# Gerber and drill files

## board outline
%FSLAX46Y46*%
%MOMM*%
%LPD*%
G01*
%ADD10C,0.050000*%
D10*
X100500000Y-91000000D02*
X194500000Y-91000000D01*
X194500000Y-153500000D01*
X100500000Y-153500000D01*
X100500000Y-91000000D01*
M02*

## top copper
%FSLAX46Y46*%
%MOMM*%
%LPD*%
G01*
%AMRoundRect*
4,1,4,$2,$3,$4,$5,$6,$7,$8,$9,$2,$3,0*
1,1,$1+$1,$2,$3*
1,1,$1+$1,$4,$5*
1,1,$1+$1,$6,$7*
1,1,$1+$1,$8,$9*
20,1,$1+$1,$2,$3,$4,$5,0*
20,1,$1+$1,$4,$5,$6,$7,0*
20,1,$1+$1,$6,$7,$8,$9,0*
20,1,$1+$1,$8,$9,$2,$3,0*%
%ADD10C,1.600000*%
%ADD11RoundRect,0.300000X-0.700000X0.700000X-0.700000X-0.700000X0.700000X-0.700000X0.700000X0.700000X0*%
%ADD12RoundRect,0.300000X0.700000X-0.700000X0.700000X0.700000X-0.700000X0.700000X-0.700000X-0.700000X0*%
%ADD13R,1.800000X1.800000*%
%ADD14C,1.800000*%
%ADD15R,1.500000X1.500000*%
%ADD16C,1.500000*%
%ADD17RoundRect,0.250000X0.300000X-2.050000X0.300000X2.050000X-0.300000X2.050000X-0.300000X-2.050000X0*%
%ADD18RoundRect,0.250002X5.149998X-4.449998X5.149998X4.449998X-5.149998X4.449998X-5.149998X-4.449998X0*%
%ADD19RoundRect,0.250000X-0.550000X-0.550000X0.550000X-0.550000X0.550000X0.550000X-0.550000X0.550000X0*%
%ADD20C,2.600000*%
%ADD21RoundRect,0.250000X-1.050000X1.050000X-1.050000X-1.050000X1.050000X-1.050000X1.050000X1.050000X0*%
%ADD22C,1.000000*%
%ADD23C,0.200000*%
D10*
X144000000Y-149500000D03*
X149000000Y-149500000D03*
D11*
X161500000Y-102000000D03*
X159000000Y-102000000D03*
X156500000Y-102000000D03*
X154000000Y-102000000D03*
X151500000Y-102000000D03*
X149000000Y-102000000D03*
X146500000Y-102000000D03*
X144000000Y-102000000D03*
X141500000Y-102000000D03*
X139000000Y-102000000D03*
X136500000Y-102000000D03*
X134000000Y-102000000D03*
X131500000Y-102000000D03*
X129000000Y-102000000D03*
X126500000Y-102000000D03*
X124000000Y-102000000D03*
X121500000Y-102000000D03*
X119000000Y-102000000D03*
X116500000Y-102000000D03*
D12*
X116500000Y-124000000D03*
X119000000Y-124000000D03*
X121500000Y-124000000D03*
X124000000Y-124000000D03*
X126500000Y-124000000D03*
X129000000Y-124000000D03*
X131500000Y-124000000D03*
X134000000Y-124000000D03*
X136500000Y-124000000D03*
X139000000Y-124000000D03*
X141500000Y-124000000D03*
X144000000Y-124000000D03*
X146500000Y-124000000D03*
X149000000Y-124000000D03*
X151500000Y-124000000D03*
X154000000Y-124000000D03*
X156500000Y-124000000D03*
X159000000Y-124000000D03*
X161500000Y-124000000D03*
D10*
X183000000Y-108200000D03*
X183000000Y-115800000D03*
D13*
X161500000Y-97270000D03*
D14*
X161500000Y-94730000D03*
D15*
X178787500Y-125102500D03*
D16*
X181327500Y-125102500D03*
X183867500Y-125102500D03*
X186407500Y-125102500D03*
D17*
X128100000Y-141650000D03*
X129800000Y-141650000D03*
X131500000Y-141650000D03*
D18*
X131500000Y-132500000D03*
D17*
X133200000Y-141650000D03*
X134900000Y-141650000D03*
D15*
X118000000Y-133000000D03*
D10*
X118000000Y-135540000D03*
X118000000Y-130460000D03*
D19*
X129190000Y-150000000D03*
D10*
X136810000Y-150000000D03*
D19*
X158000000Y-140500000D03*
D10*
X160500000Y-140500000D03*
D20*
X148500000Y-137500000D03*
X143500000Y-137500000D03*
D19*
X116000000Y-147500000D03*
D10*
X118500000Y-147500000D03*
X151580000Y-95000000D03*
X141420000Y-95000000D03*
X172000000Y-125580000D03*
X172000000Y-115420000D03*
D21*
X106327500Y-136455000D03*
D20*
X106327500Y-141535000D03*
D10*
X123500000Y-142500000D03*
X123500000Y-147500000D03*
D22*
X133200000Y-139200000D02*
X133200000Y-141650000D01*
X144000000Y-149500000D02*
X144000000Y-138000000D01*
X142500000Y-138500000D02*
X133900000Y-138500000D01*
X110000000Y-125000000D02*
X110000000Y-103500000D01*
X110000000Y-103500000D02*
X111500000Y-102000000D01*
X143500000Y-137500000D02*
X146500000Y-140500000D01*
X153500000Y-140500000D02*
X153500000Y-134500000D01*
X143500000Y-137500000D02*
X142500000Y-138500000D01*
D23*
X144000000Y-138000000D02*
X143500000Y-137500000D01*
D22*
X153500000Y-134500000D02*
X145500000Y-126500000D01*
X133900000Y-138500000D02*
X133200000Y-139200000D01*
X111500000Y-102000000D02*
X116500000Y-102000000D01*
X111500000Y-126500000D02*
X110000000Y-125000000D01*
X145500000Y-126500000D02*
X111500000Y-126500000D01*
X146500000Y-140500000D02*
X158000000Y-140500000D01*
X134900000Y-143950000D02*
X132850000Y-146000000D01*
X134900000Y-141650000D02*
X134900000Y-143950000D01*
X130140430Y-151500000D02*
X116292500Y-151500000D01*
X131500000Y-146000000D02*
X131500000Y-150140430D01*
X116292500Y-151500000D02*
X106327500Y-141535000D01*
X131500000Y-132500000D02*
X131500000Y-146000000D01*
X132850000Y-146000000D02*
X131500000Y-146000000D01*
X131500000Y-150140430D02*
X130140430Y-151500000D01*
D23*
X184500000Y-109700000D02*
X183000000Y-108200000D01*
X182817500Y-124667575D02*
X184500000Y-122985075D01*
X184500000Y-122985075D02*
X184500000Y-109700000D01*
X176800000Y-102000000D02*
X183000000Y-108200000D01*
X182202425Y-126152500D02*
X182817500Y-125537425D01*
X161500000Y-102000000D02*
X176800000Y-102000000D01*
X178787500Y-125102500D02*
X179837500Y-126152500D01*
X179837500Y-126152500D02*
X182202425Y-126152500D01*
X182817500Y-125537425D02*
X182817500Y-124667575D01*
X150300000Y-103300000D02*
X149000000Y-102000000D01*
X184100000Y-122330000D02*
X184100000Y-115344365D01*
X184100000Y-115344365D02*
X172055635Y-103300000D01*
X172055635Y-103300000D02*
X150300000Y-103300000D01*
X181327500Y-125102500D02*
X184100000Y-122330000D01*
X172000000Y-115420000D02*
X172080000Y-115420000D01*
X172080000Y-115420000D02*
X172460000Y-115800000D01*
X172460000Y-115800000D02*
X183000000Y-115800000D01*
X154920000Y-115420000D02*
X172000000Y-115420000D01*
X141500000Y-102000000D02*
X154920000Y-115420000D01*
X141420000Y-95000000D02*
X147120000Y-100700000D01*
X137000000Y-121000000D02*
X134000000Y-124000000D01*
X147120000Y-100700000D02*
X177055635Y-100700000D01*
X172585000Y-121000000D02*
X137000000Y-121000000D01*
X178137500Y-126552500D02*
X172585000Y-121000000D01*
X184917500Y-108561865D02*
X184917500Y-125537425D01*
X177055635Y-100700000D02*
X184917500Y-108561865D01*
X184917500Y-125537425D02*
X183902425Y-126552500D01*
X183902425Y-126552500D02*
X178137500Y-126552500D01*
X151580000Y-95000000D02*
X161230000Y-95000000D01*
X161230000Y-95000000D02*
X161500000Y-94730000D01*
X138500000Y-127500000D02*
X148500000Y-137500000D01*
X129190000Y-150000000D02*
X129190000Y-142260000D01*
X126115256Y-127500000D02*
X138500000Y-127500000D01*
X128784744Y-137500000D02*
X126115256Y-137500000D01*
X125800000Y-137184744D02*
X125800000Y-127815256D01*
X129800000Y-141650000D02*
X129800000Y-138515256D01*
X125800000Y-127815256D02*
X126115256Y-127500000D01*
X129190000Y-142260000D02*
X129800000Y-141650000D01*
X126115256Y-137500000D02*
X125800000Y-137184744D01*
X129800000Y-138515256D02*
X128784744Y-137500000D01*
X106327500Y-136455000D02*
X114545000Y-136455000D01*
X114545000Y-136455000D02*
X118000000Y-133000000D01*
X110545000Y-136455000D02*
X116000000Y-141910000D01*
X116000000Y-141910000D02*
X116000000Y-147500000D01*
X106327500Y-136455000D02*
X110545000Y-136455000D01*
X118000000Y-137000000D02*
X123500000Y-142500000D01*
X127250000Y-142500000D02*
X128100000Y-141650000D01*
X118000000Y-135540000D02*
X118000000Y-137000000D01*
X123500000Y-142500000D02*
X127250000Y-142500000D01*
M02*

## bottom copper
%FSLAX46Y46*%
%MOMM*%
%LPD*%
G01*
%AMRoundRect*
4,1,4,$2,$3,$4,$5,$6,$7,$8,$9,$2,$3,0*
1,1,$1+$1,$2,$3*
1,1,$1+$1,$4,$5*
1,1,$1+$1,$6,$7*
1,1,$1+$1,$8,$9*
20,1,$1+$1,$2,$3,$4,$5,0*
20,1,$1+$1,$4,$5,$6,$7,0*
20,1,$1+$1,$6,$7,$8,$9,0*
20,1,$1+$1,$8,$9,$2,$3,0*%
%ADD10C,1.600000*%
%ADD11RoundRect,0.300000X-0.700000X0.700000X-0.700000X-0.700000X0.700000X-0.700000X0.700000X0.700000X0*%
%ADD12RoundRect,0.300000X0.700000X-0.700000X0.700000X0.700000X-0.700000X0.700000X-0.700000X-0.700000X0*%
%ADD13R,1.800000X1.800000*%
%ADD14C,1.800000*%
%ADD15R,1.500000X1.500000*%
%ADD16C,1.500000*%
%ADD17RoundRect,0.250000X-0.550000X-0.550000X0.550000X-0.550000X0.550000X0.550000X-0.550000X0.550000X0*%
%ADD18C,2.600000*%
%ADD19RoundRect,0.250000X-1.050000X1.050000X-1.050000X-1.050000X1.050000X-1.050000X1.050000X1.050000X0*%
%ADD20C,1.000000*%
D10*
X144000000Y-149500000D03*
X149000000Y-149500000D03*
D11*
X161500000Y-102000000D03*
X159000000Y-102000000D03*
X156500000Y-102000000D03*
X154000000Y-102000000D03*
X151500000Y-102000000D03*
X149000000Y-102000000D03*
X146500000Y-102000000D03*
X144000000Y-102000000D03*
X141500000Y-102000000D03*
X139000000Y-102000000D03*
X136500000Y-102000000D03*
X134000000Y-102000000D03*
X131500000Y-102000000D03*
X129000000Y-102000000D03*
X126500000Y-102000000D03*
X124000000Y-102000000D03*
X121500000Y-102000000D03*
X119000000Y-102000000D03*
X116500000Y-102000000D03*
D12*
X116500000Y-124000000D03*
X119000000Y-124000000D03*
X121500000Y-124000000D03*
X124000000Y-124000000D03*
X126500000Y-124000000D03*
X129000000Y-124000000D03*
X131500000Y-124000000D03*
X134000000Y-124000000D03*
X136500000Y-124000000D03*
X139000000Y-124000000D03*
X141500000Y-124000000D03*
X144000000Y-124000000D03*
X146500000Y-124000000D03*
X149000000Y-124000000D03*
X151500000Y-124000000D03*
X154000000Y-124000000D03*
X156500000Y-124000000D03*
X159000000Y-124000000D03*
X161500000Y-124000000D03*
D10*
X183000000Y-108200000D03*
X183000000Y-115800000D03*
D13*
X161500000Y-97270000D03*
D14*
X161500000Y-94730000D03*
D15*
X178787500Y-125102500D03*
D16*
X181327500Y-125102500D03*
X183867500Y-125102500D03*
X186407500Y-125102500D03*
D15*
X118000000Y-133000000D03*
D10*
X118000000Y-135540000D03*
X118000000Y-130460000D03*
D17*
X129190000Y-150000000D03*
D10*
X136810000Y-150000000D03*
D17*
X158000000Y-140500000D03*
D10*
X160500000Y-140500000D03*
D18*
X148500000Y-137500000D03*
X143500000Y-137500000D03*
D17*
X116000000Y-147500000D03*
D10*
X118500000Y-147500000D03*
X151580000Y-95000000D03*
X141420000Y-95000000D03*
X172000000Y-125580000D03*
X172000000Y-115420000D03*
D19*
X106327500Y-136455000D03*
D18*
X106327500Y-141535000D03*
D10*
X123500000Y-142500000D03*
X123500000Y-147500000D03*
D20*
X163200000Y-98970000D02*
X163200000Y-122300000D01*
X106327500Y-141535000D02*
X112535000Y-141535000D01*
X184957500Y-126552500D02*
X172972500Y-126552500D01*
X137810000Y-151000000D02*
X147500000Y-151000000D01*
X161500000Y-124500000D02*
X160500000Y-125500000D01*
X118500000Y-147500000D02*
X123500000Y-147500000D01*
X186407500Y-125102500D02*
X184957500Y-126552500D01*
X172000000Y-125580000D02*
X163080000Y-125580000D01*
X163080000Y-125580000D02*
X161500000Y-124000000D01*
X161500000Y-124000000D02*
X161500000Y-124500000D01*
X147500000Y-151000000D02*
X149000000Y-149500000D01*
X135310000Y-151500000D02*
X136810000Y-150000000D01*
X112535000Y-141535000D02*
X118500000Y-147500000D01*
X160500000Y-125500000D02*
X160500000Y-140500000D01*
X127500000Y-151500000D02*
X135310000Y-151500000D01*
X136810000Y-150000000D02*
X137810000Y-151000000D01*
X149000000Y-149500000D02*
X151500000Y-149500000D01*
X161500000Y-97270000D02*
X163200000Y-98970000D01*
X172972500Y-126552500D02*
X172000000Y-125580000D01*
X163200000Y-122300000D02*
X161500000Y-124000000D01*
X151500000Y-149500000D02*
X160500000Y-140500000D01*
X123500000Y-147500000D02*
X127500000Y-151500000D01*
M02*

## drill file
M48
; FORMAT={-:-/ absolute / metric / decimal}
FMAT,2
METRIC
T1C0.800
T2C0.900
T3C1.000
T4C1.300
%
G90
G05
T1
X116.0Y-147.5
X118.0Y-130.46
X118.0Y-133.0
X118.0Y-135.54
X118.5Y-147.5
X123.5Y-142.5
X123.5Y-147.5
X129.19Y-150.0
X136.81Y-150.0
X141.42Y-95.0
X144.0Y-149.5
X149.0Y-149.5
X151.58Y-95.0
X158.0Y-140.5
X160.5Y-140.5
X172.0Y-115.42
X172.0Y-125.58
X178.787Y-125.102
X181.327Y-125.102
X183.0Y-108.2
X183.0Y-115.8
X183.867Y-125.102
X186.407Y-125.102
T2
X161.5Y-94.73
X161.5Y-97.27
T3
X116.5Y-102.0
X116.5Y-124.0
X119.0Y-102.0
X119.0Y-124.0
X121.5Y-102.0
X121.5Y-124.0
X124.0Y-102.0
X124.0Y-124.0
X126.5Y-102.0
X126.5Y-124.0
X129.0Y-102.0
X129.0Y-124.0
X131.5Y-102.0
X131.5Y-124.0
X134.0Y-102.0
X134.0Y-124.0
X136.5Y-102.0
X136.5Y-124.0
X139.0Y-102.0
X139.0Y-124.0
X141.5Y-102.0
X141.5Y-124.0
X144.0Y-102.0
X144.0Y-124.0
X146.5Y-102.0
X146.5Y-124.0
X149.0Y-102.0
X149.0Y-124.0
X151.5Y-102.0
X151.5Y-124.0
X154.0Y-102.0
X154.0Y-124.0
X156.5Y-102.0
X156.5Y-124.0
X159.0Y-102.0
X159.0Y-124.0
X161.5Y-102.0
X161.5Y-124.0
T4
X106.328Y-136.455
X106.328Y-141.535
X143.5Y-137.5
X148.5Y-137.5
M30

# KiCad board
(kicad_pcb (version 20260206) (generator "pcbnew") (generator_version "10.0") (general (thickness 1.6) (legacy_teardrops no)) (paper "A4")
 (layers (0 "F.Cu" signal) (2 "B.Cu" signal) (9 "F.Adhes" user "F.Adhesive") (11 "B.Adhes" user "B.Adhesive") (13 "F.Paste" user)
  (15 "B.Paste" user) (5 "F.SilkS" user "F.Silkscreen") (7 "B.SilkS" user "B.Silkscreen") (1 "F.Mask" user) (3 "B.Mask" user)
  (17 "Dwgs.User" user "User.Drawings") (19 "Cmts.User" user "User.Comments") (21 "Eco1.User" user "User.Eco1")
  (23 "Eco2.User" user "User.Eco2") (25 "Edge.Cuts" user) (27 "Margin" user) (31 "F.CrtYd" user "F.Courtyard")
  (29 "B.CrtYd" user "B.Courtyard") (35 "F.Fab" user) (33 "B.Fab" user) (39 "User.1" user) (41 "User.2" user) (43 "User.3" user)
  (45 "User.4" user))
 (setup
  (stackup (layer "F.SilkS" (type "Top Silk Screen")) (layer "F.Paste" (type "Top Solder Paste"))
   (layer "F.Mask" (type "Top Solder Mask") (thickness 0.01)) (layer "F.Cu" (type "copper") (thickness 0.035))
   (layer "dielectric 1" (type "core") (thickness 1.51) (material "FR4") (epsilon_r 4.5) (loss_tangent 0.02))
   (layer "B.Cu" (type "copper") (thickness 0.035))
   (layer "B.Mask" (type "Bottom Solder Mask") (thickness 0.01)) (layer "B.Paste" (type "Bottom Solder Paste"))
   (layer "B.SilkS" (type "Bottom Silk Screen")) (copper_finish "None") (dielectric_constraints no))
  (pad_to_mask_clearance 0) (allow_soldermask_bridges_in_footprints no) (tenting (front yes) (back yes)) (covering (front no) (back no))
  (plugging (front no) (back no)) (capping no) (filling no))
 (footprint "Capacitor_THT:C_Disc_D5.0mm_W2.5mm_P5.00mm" (layer "F.Cu") (at 144 149.5)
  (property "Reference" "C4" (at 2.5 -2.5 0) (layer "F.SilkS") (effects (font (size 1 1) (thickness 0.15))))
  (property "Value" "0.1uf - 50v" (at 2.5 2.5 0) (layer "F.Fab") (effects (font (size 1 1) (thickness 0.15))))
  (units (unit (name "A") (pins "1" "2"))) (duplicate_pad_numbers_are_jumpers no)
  (pad "1" thru_hole circle (at 0 0) (size 1.6 1.6) (drill 0.8) (layers "*.Cu" "*.Mask") (remove_unused_layers no) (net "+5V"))
  (pad "2" thru_hole circle (at 5 0) (size 1.6 1.6) (drill 0.8) (layers "*.Cu" "*.Mask") (remove_unused_layers no) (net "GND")))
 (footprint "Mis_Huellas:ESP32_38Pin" (layer "F.Cu") (at 162.5 113 -90)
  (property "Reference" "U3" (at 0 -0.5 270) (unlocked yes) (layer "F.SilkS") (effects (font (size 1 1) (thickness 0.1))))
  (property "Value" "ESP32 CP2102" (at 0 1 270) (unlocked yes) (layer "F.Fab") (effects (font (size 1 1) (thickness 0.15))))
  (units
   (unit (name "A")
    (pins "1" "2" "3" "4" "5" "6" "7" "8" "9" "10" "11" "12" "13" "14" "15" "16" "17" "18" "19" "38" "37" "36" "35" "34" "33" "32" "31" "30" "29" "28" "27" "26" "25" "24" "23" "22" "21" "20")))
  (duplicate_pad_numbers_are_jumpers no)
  (pad "1" thru_hole roundrect (at -11 1 270) (size 2 2) (drill 1) (layers "*.Cu" "*.Mask") (remove_unused_layers no)
   (roundrect_rratio 0.15) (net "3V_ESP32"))
  (pad "2" thru_hole roundrect (at -11 3.5 270) (size 2 2) (drill 1) (layers "*.Cu" "*.Mask") (remove_unused_layers no)
   (roundrect_rratio 0.15) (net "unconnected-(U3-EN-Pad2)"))
  (pad "3" thru_hole roundrect (at -11 6 270) (size 2 2) (drill 1) (layers "*.Cu" "*.Mask") (remove_unused_layers no)
   (roundrect_rratio 0.15) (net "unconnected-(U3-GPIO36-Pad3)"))
  (pad "4" thru_hole roundrect (at -11 8.5 270) (size 2 2) (drill 1) (layers "*.Cu" "*.Mask") (remove_unused_layers no)
   (roundrect_rratio 0.15) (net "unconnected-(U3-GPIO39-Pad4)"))
  (pad "5" thru_hole roundrect (at -11 11 270) (size 2 2) (drill 1) (layers "*.Cu" "*.Mask") (remove_unused_layers no)
   (roundrect_rratio 0.15) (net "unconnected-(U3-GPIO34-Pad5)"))
  (pad "6" thru_hole roundrect (at -11 13.5 270) (size 2 2) (drill 1) (layers "*.Cu" "*.Mask") (remove_unused_layers no)
   (roundrect_rratio 0.15) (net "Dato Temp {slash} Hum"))
  (pad "7" thru_hole roundrect (at -11 16 270) (size 2 2) (drill 1) (layers "*.Cu" "*.Mask") (remove_unused_layers no)
   (roundrect_rratio 0.15) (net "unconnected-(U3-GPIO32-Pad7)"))
  (pad "8" thru_hole roundrect (at -11 18.5 270) (size 2 2) (drill 1) (layers "*.Cu" "*.Mask") (remove_unused_layers no)
   (roundrect_rratio 0.15) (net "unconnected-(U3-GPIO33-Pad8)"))
  (pad "9" thru_hole roundrect (at -11 21 270) (size 2 2) (drill 1) (layers "*.Cu" "*.Mask") (remove_unused_layers no)
   (roundrect_rratio 0.15) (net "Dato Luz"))
  (pad "10" thru_hole roundrect (at -11 23.5 270) (size 2 2) (drill 1) (layers "*.Cu" "*.Mask") (remove_unused_layers no)
   (roundrect_rratio 0.15) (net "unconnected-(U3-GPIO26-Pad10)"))
  (pad "11" thru_hole roundrect (at -11 26 270) (size 2 2) (drill 1) (layers "*.Cu" "*.Mask") (remove_unused_layers no)
   (roundrect_rratio 0.15) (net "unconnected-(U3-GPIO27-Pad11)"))
  (pad "12" thru_hole roundrect (at -11 28.5 270) (size 2 2) (drill 1) (layers "*.Cu" "*.Mask") (remove_unused_layers no)
   (roundrect_rratio 0.15) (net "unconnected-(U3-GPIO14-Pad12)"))
  (pad "13" thru_hole roundrect (at -11 31 270) (size 2 2) (drill 1) (layers "*.Cu" "*.Mask") (remove_unused_layers no)
   (roundrect_rratio 0.15) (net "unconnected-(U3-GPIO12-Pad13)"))
  (pad "14" thru_hole roundrect (at -11 33.5 270) (size 2 2) (drill 1) (layers "*.Cu" "*.Mask") (remove_unused_layers no)
   (roundrect_rratio 0.15) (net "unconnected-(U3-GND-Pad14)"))
  (pad "15" thru_hole roundrect (at -11 36 270) (size 2 2) (drill 1) (layers "*.Cu" "*.Mask") (remove_unused_layers no)
   (roundrect_rratio 0.15) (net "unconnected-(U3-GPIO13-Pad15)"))
  (pad "16" thru_hole roundrect (at -11 38.5 270) (size 2 2) (drill 1) (layers "*.Cu" "*.Mask") (remove_unused_layers no)
   (roundrect_rratio 0.15) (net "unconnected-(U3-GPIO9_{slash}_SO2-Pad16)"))
  (pad "17" thru_hole roundrect (at -11 41 270) (size 2 2) (drill 1) (layers "*.Cu" "*.Mask") (remove_unused_layers no)
   (roundrect_rratio 0.15) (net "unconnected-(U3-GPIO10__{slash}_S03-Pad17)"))
  (pad "18" thru_hole roundrect (at -11 43.5 270) (size 2 2) (drill 1) (layers "*.Cu" "*.Mask") (remove_unused_layers no)
   (roundrect_rratio 0.15) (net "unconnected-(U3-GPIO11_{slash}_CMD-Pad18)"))
  (pad "19" thru_hole roundrect (at -11 46 270) (size 2 2) (drill 1) (layers "*.Cu" "*.Mask") (remove_unused_layers no)
   (roundrect_rratio 0.15) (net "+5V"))
  (pad "20" thru_hole roundrect (at 11 46 90) (size 2 2) (drill 1) (layers "*.Cu" "*.Mask") (remove_unused_layers no)
   (roundrect_rratio 0.15) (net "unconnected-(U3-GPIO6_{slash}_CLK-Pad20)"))
  (pad "21" thru_hole roundrect (at 11 43.5 90) (size 2 2) (drill 1) (layers "*.Cu" "*.Mask") (remove_unused_layers no)
   (roundrect_rratio 0.15) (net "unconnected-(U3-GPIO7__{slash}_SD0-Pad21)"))
  (pad "22" thru_hole roundrect (at 11 41 90) (size 2 2) (drill 1) (layers "*.Cu" "*.Mask") (remove_unused_layers no)
   (roundrect_rratio 0.15) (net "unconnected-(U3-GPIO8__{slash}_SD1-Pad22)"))
  (pad "23" thru_hole roundrect (at 11 38.5 90) (size 2 2) (drill 1) (layers "*.Cu" "*.Mask") (remove_unused_layers no)
   (roundrect_rratio 0.15) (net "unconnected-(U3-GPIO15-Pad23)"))
  (pad "24" thru_hole roundrect (at 11 36 90) (size 2 2) (drill 1) (layers "*.Cu" "*.Mask") (remove_unused_layers no)
   (roundrect_rratio 0.15) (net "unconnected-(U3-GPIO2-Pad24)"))
  (pad "25" thru_hole roundrect (at 11 33.5 90) (size 2 2) (drill 1) (layers "*.Cu" "*.Mask") (remove_unused_layers no)
   (roundrect_rratio 0.15) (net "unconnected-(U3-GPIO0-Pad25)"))
  (pad "26" thru_hole roundrect (at 11 31 90) (size 2 2) (drill 1) (layers "*.Cu" "*.Mask") (remove_unused_layers no)
   (roundrect_rratio 0.15) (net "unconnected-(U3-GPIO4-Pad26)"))
  (pad "27" thru_hole roundrect (at 11 28.5 90) (size 2 2) (drill 1) (layers "*.Cu" "*.Mask") (remove_unused_layers no)
   (roundrect_rratio 0.15) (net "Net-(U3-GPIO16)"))
  (pad "28" thru_hole roundrect (at 11 26 90) (size 2 2) (drill 1) (layers "*.Cu" "*.Mask") (remove_unused_layers no)
   (roundrect_rratio 0.15) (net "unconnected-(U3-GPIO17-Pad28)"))
  (pad "29" thru_hole roundrect (at 11 23.5 90) (size 2 2) (drill 1) (layers "*.Cu" "*.Mask") (remove_unused_layers no)
   (roundrect_rratio 0.15) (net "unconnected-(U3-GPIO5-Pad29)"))
  (pad "30" thru_hole roundrect (at 11 21 90) (size 2 2) (drill 1) (layers "*.Cu" "*.Mask") (remove_unused_layers no)
   (roundrect_rratio 0.15) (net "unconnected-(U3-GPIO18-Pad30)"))
  (pad "31" thru_hole roundrect (at 11 18.5 90) (size 2 2) (drill 1) (layers "*.Cu" "*.Mask") (remove_unused_layers no)
   (roundrect_rratio 0.15) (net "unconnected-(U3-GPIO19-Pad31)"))
  (pad "32" thru_hole roundrect (at 11 16 90) (size 2 2) (drill 1) (layers "*.Cu" "*.Mask") (remove_unused_layers no)
   (roundrect_rratio 0.15) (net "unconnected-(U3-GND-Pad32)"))
  (pad "33" thru_hole roundrect (at 11 13.5 90) (size 2 2) (drill 1) (layers "*.Cu" "*.Mask") (remove_unused_layers no)
   (roundrect_rratio 0.15) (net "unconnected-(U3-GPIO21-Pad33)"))
  (pad "34" thru_hole roundrect (at 11 11 90) (size 2 2) (drill 1) (layers "*.Cu" "*.Mask") (remove_unused_layers no)
   (roundrect_rratio 0.15) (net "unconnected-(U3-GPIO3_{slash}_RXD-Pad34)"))
  (pad "35" thru_hole roundrect (at 11 8.5 90) (size 2 2) (drill 1) (layers "*.Cu" "*.Mask") (remove_unused_layers no)
   (roundrect_rratio 0.15) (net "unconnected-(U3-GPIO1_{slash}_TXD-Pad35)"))
  (pad "36" thru_hole roundrect (at 11 6 90) (size 2 2) (drill 1) (layers "*.Cu" "*.Mask") (remove_unused_layers no) (roundrect_rratio 0.15)
   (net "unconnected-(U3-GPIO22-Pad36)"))
  (pad "37" thru_hole roundrect (at 11 3.5 90) (size 2 2) (drill 1) (layers "*.Cu" "*.Mask") (remove_unused_layers no)
   (roundrect_rratio 0.15) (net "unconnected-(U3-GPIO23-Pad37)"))
  (pad "38" thru_hole roundrect (at 11 1 90) (size 2 2) (drill 1) (layers "*.Cu" "*.Mask") (remove_unused_layers no) (roundrect_rratio 0.15)
   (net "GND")))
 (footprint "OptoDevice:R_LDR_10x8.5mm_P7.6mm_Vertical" (layer "F.Cu") (at 183 108.2 -90)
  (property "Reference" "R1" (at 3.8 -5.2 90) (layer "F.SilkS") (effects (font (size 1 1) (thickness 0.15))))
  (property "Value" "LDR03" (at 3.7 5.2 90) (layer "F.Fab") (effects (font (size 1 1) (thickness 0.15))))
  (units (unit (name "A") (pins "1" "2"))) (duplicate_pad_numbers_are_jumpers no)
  (pad "1" thru_hole circle (at 0 0 270) (size 1.6 1.6) (drill 0.8) (layers "*.Cu" "*.Mask") (remove_unused_layers no) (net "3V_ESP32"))
  (pad "2" thru_hole circle (at 7.6 0 270) (size 1.6 1.6) (drill 0.8) (layers "*.Cu" "*.Mask") (remove_unused_layers no) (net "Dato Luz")))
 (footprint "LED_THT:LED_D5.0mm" (layer "F.Cu") (at 161.5 97.27 90)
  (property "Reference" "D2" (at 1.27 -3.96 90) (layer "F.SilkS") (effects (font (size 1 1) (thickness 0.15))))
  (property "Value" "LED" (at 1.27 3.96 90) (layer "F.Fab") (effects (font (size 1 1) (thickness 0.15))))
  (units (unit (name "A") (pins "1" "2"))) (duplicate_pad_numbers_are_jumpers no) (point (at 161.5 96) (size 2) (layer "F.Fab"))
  (pad "1" thru_hole rect (at 0 0 90) (size 1.8 1.8) (drill 0.9) (layers "*.Cu" "*.Mask") (remove_unused_layers no) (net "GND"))
  (pad "2" thru_hole circle (at 2.54 0 90) (size 1.8 1.8) (drill 0.9) (layers "*.Cu" "*.Mask") (remove_unused_layers no)
   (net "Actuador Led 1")))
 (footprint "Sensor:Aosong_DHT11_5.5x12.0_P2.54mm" (layer "F.Cu") (at 178.7875 125.1025 90)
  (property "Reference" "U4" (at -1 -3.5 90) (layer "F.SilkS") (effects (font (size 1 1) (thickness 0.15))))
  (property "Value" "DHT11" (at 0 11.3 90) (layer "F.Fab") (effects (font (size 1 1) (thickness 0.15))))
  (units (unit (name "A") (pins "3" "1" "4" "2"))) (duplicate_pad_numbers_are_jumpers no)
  (pad "1" thru_hole rect (at 0 0 90) (size 1.5 1.5) (drill 0.8) (layers "*.Cu" "*.Mask") (remove_unused_layers no) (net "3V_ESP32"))
  (pad "2" thru_hole circle (at 0 2.54 90) (size 1.5 1.5) (drill 0.8) (layers "*.Cu" "*.Mask") (remove_unused_layers no)
   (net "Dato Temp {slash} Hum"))
  (pad "3" thru_hole circle (at 0 5.08 90) (size 1.5 1.5) (drill 0.8) (layers "*.Cu" "*.Mask") (remove_unused_layers no)
   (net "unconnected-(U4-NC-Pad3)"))
  (pad "4" thru_hole circle (at 0 7.62 90) (size 1.5 1.5) (drill 0.8) (layers "*.Cu" "*.Mask") (remove_unused_layers no) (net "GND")))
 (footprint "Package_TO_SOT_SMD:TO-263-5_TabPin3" (layer "F.Cu") (at 131.5 134 90)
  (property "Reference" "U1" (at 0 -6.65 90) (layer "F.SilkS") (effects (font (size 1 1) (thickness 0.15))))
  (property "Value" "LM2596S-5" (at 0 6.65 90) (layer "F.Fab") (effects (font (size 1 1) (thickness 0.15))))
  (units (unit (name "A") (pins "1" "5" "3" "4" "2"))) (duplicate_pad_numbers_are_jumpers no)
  (pad "" smd roundrect (at -0.925 -2.775 90) (size 4.55 5.25) (layers "F.Paste") (roundrect_rratio 0.054945))
  (pad "" smd roundrect (at -0.925 2.775 90) (size 4.55 5.25) (layers "F.Paste") (roundrect_rratio 0.054945))
  (pad "" smd roundrect (at 3.925 -2.775 90) (size 4.55 5.25) (layers "F.Paste") (roundrect_rratio 0.054945))
  (pad "" smd roundrect (at 3.925 2.775 90) (size 4.55 5.25) (layers "F.Paste") (roundrect_rratio 0.054945))
  (pad "1" smd roundrect (at -7.65 -3.4 90) (size 4.6 1.1) (layers "F.Cu" "F.Mask" "F.Paste") (roundrect_rratio 0.227273)
   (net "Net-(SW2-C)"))
  (pad "2" smd roundrect (at -7.65 -1.7 90) (size 4.6 1.1) (layers "F.Cu" "F.Mask" "F.Paste") (roundrect_rratio 0.227273) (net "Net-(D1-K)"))
  (pad "3" smd roundrect (at -7.65 0 90) (size 4.6 1.1) (layers "F.Cu" "F.Mask" "F.Paste") (roundrect_rratio 0.227273) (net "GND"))
  (pad "3" smd roundrect (at 1.5 0 90) (size 9.4 10.8) (layers "F.Cu" "F.Mask") (roundrect_rratio 0.026596) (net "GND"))
  (pad "4" smd roundrect (at -7.65 1.7 90) (size 4.6 1.1) (layers "F.Cu" "F.Mask" "F.Paste") (roundrect_rratio 0.227273) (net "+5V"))
  (pad "5" smd roundrect (at -7.65 3.4 90) (size 4.6 1.1) (layers "F.Cu" "F.Mask" "F.Paste") (roundrect_rratio 0.227273) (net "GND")))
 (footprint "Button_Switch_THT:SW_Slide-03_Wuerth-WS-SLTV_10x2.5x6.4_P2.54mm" (layer "F.Cu") (at 118 133 90)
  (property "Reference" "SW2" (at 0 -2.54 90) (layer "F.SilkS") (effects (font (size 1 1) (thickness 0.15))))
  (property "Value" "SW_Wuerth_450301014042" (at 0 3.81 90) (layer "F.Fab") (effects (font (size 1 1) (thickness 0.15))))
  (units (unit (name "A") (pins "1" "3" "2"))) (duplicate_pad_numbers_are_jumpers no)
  (pad "1" thru_hole rect (at 0 0 90) (size 1.5 1.5) (drill 0.8) (layers "*.Cu" "*.Mask") (remove_unused_layers no) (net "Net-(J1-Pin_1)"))
  (pad "2" thru_hole circle (at -2.54 0 90) (size 1.6 1.6) (drill 0.8) (layers "*.Cu" "*.Mask") (remove_unused_layers no)
   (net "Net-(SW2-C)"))
  (pad "3" thru_hole circle (at 2.54 0 90) (size 1.6 1.6) (drill 0.8) (layers "*.Cu" "*.Mask") (remove_unused_layers no)
   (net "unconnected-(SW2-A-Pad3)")))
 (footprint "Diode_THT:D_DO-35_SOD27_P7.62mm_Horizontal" (layer "F.Cu") (at 129.19 150)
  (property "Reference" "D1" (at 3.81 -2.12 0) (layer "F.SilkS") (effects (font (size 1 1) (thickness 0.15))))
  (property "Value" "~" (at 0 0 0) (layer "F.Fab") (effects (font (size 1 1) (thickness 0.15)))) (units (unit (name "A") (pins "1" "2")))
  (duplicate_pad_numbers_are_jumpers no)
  (pad "1" thru_hole roundrect (at 0 0) (size 1.6 1.6) (drill 0.8) (layers "*.Cu" "*.Mask") (remove_unused_layers no)
   (roundrect_rratio 0.15625) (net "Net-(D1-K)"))
  (pad "2" thru_hole circle (at 7.62 0) (size 1.6 1.6) (drill 0.8) (layers "*.Cu" "*.Mask") (remove_unused_layers no) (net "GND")))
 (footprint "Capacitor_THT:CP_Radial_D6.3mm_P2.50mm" (layer "F.Cu") (at 158 140.5)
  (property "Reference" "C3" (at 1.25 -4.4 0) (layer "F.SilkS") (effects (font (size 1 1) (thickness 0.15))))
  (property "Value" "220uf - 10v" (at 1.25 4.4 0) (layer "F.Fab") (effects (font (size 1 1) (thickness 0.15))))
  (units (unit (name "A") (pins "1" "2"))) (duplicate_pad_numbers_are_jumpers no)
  (pad "1" thru_hole roundrect (at 0 0) (size 1.6 1.6) (drill 0.8) (layers "*.Cu" "*.Mask") (remove_unused_layers no)
   (roundrect_rratio 0.15625) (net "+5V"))
  (pad "2" thru_hole circle (at 2.5 0) (size 1.6 1.6) (drill 0.8) (layers "*.Cu" "*.Mask") (remove_unused_layers no) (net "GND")))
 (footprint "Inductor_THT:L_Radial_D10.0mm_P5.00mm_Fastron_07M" (layer "F.Cu") (at 148.5 137.5 180)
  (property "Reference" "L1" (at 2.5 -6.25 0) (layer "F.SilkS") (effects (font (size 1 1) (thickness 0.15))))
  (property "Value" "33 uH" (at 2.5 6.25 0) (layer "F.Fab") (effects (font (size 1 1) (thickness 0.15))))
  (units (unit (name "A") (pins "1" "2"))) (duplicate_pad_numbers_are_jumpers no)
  (pad "1" thru_hole circle (at 0 0 180) (size 2.6 2.6) (drill 1.3) (layers "*.Cu" "*.Mask") (remove_unused_layers no) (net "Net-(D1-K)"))
  (pad "2" thru_hole circle (at 5 0 180) (size 2.6 2.6) (drill 1.3) (layers "*.Cu" "*.Mask") (remove_unused_layers no) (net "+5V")))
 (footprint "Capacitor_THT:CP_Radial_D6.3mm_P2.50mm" (layer "F.Cu") (at 116 147.5)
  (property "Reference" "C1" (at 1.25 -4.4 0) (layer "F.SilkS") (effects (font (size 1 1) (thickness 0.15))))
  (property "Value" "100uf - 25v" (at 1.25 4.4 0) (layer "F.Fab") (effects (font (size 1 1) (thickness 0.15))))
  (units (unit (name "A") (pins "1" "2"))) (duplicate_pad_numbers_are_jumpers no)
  (pad "1" thru_hole roundrect (at 0 0) (size 1.6 1.6) (drill 0.8) (layers "*.Cu" "*.Mask") (remove_unused_layers no)
   (roundrect_rratio 0.15625) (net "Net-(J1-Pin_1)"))
  (pad "2" thru_hole circle (at 2.5 0) (size 1.6 1.6) (drill 0.8) (layers "*.Cu" "*.Mask") (remove_unused_layers no) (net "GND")))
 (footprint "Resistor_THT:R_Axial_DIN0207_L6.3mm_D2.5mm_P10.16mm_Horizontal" (layer "F.Cu") (at 151.58 95 180)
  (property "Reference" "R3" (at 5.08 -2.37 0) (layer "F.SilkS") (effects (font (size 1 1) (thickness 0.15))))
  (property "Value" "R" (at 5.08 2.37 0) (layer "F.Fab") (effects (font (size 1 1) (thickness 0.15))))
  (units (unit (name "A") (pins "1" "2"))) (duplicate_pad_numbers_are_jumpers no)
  (pad "1" thru_hole circle (at 0 0 180) (size 1.6 1.6) (drill 0.8) (layers "*.Cu" "*.Mask") (remove_unused_layers no)
   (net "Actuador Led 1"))
  (pad "2" thru_hole circle (at 10.16 0 180) (size 1.6 1.6) (drill 0.8) (layers "*.Cu" "*.Mask") (remove_unused_layers no)
   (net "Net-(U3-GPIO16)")))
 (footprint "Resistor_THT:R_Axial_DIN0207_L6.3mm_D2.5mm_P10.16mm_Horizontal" (layer "F.Cu") (at 172 125.58 90)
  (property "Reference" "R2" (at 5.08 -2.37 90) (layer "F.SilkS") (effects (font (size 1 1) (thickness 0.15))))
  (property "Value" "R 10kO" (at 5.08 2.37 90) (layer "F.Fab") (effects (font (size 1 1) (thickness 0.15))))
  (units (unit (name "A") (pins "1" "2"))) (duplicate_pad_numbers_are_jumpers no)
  (pad "1" thru_hole circle (at 0 0 90) (size 1.6 1.6) (drill 0.8) (layers "*.Cu" "*.Mask") (remove_unused_layers no) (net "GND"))
  (pad "2" thru_hole circle (at 10.16 0 90) (size 1.6 1.6) (drill 0.8) (layers "*.Cu" "*.Mask") (remove_unused_layers no) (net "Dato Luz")))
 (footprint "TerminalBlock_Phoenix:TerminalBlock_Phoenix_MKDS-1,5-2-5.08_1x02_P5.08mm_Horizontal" (layer "F.Cu") (at 106.3275 136.455 -90)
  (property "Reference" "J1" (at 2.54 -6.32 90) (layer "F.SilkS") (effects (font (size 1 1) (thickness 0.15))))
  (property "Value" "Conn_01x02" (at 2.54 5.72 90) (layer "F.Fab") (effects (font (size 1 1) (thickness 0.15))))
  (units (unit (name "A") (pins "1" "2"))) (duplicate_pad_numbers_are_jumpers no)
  (pad "1" thru_hole roundrect (at 0 0 270) (size 2.6 2.6) (drill 1.3) (layers "*.Cu" "*.Mask") (remove_unused_layers no)
   (roundrect_rratio 0.096154) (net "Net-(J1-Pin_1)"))
  (pad "2" thru_hole circle (at 5.08 0 270) (size 2.6 2.6) (drill 1.3) (layers "*.Cu" "*.Mask") (remove_unused_layers no) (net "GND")))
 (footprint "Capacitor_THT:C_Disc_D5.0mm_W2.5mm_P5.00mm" (layer "F.Cu") (at 123.5 142.5 -90)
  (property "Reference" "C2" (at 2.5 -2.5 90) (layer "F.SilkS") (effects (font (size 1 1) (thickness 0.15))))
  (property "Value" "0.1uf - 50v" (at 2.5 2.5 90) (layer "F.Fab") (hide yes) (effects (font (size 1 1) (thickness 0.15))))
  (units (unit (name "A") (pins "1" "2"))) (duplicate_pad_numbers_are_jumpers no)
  (pad "1" thru_hole circle (at 0 0 270) (size 1.6 1.6) (drill 0.8) (layers "*.Cu" "*.Mask") (remove_unused_layers no) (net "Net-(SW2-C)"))
  (pad "2" thru_hole circle (at 5 0 270) (size 1.6 1.6) (drill 0.8) (layers "*.Cu" "*.Mask") (remove_unused_layers no) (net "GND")))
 (gr_rect (start 100.5 91) (end 194.5 153.5) (stroke (width 0.05) (type default)) (fill no) (layer "Edge.Cuts"))
 (segment (start 133.2 139.2) (end 133.2 141.65) (width 1) (layer "F.Cu") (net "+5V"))
 (segment (start 144 149.5) (end 144 138) (width 1) (layer "F.Cu") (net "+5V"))
 (segment (start 142.5 138.5) (end 133.9 138.5) (width 1) (layer "F.Cu") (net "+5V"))
 (segment (start 110 125) (end 110 103.5) (width 1) (layer "F.Cu") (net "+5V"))
 (segment (start 110 103.5) (end 111.5 102) (width 1) (layer "F.Cu") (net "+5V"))
 (segment (start 143.5 137.5) (end 146.5 140.5) (width 1) (layer "F.Cu") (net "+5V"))
 (segment (start 153.5 140.5) (end 153.5 134.5) (width 1) (layer "F.Cu") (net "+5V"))
 (segment (start 143.5 137.5) (end 142.5 138.5) (width 1) (layer "F.Cu") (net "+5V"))
 (segment (start 144 138) (end 143.5 137.5) (width 0.2) (layer "F.Cu") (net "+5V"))
 (segment (start 153.5 134.5) (end 145.5 126.5) (width 1) (layer "F.Cu") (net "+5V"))
 (segment (start 133.9 138.5) (end 133.2 139.2) (width 1) (layer "F.Cu") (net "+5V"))
 (segment (start 111.5 102) (end 116.5 102) (width 1) (layer "F.Cu") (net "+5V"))
 (segment (start 111.5 126.5) (end 110 125) (width 1) (layer "F.Cu") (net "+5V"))
 (segment (start 145.5 126.5) (end 111.5 126.5) (width 1) (layer "F.Cu") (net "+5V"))
 (segment (start 146.5 140.5) (end 158 140.5) (width 1) (layer "F.Cu") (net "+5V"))
 (segment (start 134.9 143.95) (end 132.85 146) (width 1) (layer "F.Cu") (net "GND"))
 (segment (start 134.9 141.65) (end 134.9 143.95) (width 1) (layer "F.Cu") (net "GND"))
 (segment (start 130.14043 151.5) (end 116.2925 151.5) (width 1) (layer "F.Cu") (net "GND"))
 (segment (start 131.5 146) (end 131.5 150.14043) (width 1) (layer "F.Cu") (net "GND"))
 (segment (start 116.2925 151.5) (end 106.3275 141.535) (width 1) (layer "F.Cu") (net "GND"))
 (segment (start 131.5 132.5) (end 131.5 146) (width 1) (layer "F.Cu") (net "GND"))
 (segment (start 132.85 146) (end 131.5 146) (width 1) (layer "F.Cu") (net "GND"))
 (segment (start 131.5 150.14043) (end 130.14043 151.5) (width 1) (layer "F.Cu") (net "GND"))
 (segment (start 163.2 98.97) (end 163.2 122.3) (width 1) (layer "B.Cu") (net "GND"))
 (segment (start 106.3275 141.535) (end 112.535 141.535) (width 1) (layer "B.Cu") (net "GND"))
 (segment (start 184.9575 126.5525) (end 172.9725 126.5525) (width 1) (layer "B.Cu") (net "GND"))
 (segment (start 137.81 151) (end 147.5 151) (width 1) (layer "B.Cu") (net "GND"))
 (segment (start 161.5 124.5) (end 160.5 125.5) (width 1) (layer "B.Cu") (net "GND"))
 (segment (start 118.5 147.5) (end 123.5 147.5) (width 1) (layer "B.Cu") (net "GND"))
 (segment (start 186.4075 125.1025) (end 184.9575 126.5525) (width 1) (layer "B.Cu") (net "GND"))
 (segment (start 172 125.58) (end 163.08 125.58) (width 1) (layer "B.Cu") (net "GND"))
 (segment (start 163.08 125.58) (end 161.5 124) (width 1) (layer "B.Cu") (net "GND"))
 (segment (start 161.5 124) (end 161.5 124.5) (width 1) (layer "B.Cu") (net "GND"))
 (segment (start 147.5 151) (end 149 149.5) (width 1) (layer "B.Cu") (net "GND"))
 (segment (start 135.31 151.5) (end 136.81 150) (width 1) (layer "B.Cu") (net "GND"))
 (segment (start 112.535 141.535) (end 118.5 147.5) (width 1) (layer "B.Cu") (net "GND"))
 (segment (start 160.5 125.5) (end 160.5 140.5) (width 1) (layer "B.Cu") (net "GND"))
 (segment (start 127.5 151.5) (end 135.31 151.5) (width 1) (layer "B.Cu") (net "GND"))
 (segment (start 136.81 150) (end 137.81 151) (width 1) (layer "B.Cu") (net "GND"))
 (segment (start 149 149.5) (end 151.5 149.5) (width 1) (layer "B.Cu") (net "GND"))
 (segment (start 161.5 97.27) (end 163.2 98.97) (width 1) (layer "B.Cu") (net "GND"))
 (segment (start 172.9725 126.5525) (end 172 125.58) (width 1) (layer "B.Cu") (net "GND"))
 (segment (start 163.2 122.3) (end 161.5 124) (width 1) (layer "B.Cu") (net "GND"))
 (segment (start 151.5 149.5) (end 160.5 140.5) (width 1) (layer "B.Cu") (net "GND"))
 (segment (start 123.5 147.5) (end 127.5 151.5) (width 1) (layer "B.Cu") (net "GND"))
 (segment (start 184.5 109.7) (end 183 108.2) (width 0.2) (layer "F.Cu") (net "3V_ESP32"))
 (segment (start 182.8175 124.667575) (end 184.5 122.985075) (width 0.2) (layer "F.Cu") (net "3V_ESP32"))
 (segment (start 184.5 122.985075) (end 184.5 109.7) (width 0.2) (layer "F.Cu") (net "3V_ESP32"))
 (segment (start 176.8 102) (end 183 108.2) (width 0.2) (layer "F.Cu") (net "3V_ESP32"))
 (segment (start 182.202425 126.1525) (end 182.8175 125.537425) (width 0.2) (layer "F.Cu") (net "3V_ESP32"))
 (segment (start 161.5 102) (end 176.8 102) (width 0.2) (layer "F.Cu") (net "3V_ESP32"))
 (segment (start 178.7875 125.1025) (end 179.8375 126.1525) (width 0.2) (layer "F.Cu") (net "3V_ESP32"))
 (segment (start 179.8375 126.1525) (end 182.202425 126.1525) (width 0.2) (layer "F.Cu") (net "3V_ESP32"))
 (segment (start 182.8175 125.537425) (end 182.8175 124.667575) (width 0.2) (layer "F.Cu") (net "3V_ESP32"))
 (segment (start 150.3 103.3) (end 149 102) (width 0.2) (layer "F.Cu") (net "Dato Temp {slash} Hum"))
 (segment (start 184.1 122.33) (end 184.1 115.344365) (width 0.2) (layer "F.Cu") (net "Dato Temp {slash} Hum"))
 (segment (start 184.1 115.344365) (end 172.055635 103.3) (width 0.2) (layer "F.Cu") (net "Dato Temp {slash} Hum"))
 (segment (start 172.055635 103.3) (end 150.3 103.3) (width 0.2) (layer "F.Cu") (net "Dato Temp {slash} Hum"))
 (segment (start 181.3275 125.1025) (end 184.1 122.33) (width 0.2) (layer "F.Cu") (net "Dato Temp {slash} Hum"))
 (segment (start 172 115.42) (end 172.08 115.42) (width 0.2) (layer "F.Cu") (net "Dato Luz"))
 (segment (start 172.08 115.42) (end 172.46 115.8) (width 0.2) (layer "F.Cu") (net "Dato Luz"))
 (segment (start 172.46 115.8) (end 183 115.8) (width 0.2) (layer "F.Cu") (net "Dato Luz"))
 (segment (start 154.92 115.42) (end 172 115.42) (width 0.2) (layer "F.Cu") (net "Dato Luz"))
 (segment (start 141.5 102) (end 154.92 115.42) (width 0.2) (layer "F.Cu") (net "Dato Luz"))
 (segment (start 141.42 95) (end 147.12 100.7) (width 0.2) (layer "F.Cu") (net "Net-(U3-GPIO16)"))
 (segment (start 137 121) (end 134 124) (width 0.2) (layer "F.Cu") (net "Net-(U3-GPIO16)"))
 (segment (start 147.12 100.7) (end 177.055635 100.7) (width 0.2) (layer "F.Cu") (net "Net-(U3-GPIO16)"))
 (segment (start 172.585 121) (end 137 121) (width 0.2) (layer "F.Cu") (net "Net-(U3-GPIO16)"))
 (segment (start 178.1375 126.5525) (end 172.585 121) (width 0.2) (layer "F.Cu") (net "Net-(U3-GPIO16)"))
 (segment (start 184.9175 108.561865) (end 184.9175 125.537425) (width 0.2) (layer "F.Cu") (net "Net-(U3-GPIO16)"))
 (segment (start 177.055635 100.7) (end 184.9175 108.561865) (width 0.2) (layer "F.Cu") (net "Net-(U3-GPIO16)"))
 (segment (start 184.9175 125.537425) (end 183.902425 126.5525) (width 0.2) (layer "F.Cu") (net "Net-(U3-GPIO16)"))
 (segment (start 183.902425 126.5525) (end 178.1375 126.5525) (width 0.2) (layer "F.Cu") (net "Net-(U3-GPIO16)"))
 (segment (start 151.58 95) (end 161.23 95) (width 0.2) (layer "F.Cu") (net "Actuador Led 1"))
 (segment (start 161.23 95) (end 161.5 94.73) (width 0.2) (layer "F.Cu") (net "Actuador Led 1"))
 (segment (start 138.5 127.5) (end 148.5 137.5) (width 0.2) (layer "F.Cu") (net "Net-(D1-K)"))
 (segment (start 129.19 150) (end 129.19 142.26) (width 0.2) (layer "F.Cu") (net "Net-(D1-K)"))
 (segment (start 126.115256 127.5) (end 138.5 127.5) (width 0.2) (layer "F.Cu") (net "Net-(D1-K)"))
 (segment (start 128.784744 137.5) (end 126.115256 137.5) (width 0.2) (layer "F.Cu") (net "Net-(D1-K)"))
 (segment (start 125.8 137.184744) (end 125.8 127.815256) (width 0.2) (layer "F.Cu") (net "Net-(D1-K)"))
 (segment (start 129.8 141.65) (end 129.8 138.515256) (width 0.2) (layer "F.Cu") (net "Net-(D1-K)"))
 (segment (start 125.8 127.815256) (end 126.115256 127.5) (width 0.2) (layer "F.Cu") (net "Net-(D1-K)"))
 (segment (start 129.19 142.26) (end 129.8 141.65) (width 0.2) (layer "F.Cu") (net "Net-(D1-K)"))
 (segment (start 126.115256 137.5) (end 125.8 137.184744) (width 0.2) (layer "F.Cu") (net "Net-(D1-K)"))
 (segment (start 129.8 138.515256) (end 128.784744 137.5) (width 0.2) (layer "F.Cu") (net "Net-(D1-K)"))
 (segment (start 106.3275 136.455) (end 114.545 136.455) (width 0.2) (layer "F.Cu") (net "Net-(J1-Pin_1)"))
 (segment (start 114.545 136.455) (end 118 133) (width 0.2) (layer "F.Cu") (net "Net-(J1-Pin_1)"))
 (segment (start 110.545 136.455) (end 116 141.91) (width 0.2) (layer "F.Cu") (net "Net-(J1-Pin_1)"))
 (segment (start 116 141.91) (end 116 147.5) (width 0.2) (layer "F.Cu") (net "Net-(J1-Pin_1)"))
 (segment (start 106.3275 136.455) (end 110.545 136.455) (width 0.2) (layer "F.Cu") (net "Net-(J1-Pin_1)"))
 (segment (start 118 137) (end 123.5 142.5) (width 0.2) (layer "F.Cu") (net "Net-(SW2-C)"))
 (segment (start 127.25 142.5) (end 128.1 141.65) (width 0.2) (layer "F.Cu") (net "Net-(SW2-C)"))
 (segment (start 118 135.54) (end 118 137) (width 0.2) (layer "F.Cu") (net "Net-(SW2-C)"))
 (segment (start 123.5 142.5) (end 127.25 142.5) (width 0.2) (layer "F.Cu") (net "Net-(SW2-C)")))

